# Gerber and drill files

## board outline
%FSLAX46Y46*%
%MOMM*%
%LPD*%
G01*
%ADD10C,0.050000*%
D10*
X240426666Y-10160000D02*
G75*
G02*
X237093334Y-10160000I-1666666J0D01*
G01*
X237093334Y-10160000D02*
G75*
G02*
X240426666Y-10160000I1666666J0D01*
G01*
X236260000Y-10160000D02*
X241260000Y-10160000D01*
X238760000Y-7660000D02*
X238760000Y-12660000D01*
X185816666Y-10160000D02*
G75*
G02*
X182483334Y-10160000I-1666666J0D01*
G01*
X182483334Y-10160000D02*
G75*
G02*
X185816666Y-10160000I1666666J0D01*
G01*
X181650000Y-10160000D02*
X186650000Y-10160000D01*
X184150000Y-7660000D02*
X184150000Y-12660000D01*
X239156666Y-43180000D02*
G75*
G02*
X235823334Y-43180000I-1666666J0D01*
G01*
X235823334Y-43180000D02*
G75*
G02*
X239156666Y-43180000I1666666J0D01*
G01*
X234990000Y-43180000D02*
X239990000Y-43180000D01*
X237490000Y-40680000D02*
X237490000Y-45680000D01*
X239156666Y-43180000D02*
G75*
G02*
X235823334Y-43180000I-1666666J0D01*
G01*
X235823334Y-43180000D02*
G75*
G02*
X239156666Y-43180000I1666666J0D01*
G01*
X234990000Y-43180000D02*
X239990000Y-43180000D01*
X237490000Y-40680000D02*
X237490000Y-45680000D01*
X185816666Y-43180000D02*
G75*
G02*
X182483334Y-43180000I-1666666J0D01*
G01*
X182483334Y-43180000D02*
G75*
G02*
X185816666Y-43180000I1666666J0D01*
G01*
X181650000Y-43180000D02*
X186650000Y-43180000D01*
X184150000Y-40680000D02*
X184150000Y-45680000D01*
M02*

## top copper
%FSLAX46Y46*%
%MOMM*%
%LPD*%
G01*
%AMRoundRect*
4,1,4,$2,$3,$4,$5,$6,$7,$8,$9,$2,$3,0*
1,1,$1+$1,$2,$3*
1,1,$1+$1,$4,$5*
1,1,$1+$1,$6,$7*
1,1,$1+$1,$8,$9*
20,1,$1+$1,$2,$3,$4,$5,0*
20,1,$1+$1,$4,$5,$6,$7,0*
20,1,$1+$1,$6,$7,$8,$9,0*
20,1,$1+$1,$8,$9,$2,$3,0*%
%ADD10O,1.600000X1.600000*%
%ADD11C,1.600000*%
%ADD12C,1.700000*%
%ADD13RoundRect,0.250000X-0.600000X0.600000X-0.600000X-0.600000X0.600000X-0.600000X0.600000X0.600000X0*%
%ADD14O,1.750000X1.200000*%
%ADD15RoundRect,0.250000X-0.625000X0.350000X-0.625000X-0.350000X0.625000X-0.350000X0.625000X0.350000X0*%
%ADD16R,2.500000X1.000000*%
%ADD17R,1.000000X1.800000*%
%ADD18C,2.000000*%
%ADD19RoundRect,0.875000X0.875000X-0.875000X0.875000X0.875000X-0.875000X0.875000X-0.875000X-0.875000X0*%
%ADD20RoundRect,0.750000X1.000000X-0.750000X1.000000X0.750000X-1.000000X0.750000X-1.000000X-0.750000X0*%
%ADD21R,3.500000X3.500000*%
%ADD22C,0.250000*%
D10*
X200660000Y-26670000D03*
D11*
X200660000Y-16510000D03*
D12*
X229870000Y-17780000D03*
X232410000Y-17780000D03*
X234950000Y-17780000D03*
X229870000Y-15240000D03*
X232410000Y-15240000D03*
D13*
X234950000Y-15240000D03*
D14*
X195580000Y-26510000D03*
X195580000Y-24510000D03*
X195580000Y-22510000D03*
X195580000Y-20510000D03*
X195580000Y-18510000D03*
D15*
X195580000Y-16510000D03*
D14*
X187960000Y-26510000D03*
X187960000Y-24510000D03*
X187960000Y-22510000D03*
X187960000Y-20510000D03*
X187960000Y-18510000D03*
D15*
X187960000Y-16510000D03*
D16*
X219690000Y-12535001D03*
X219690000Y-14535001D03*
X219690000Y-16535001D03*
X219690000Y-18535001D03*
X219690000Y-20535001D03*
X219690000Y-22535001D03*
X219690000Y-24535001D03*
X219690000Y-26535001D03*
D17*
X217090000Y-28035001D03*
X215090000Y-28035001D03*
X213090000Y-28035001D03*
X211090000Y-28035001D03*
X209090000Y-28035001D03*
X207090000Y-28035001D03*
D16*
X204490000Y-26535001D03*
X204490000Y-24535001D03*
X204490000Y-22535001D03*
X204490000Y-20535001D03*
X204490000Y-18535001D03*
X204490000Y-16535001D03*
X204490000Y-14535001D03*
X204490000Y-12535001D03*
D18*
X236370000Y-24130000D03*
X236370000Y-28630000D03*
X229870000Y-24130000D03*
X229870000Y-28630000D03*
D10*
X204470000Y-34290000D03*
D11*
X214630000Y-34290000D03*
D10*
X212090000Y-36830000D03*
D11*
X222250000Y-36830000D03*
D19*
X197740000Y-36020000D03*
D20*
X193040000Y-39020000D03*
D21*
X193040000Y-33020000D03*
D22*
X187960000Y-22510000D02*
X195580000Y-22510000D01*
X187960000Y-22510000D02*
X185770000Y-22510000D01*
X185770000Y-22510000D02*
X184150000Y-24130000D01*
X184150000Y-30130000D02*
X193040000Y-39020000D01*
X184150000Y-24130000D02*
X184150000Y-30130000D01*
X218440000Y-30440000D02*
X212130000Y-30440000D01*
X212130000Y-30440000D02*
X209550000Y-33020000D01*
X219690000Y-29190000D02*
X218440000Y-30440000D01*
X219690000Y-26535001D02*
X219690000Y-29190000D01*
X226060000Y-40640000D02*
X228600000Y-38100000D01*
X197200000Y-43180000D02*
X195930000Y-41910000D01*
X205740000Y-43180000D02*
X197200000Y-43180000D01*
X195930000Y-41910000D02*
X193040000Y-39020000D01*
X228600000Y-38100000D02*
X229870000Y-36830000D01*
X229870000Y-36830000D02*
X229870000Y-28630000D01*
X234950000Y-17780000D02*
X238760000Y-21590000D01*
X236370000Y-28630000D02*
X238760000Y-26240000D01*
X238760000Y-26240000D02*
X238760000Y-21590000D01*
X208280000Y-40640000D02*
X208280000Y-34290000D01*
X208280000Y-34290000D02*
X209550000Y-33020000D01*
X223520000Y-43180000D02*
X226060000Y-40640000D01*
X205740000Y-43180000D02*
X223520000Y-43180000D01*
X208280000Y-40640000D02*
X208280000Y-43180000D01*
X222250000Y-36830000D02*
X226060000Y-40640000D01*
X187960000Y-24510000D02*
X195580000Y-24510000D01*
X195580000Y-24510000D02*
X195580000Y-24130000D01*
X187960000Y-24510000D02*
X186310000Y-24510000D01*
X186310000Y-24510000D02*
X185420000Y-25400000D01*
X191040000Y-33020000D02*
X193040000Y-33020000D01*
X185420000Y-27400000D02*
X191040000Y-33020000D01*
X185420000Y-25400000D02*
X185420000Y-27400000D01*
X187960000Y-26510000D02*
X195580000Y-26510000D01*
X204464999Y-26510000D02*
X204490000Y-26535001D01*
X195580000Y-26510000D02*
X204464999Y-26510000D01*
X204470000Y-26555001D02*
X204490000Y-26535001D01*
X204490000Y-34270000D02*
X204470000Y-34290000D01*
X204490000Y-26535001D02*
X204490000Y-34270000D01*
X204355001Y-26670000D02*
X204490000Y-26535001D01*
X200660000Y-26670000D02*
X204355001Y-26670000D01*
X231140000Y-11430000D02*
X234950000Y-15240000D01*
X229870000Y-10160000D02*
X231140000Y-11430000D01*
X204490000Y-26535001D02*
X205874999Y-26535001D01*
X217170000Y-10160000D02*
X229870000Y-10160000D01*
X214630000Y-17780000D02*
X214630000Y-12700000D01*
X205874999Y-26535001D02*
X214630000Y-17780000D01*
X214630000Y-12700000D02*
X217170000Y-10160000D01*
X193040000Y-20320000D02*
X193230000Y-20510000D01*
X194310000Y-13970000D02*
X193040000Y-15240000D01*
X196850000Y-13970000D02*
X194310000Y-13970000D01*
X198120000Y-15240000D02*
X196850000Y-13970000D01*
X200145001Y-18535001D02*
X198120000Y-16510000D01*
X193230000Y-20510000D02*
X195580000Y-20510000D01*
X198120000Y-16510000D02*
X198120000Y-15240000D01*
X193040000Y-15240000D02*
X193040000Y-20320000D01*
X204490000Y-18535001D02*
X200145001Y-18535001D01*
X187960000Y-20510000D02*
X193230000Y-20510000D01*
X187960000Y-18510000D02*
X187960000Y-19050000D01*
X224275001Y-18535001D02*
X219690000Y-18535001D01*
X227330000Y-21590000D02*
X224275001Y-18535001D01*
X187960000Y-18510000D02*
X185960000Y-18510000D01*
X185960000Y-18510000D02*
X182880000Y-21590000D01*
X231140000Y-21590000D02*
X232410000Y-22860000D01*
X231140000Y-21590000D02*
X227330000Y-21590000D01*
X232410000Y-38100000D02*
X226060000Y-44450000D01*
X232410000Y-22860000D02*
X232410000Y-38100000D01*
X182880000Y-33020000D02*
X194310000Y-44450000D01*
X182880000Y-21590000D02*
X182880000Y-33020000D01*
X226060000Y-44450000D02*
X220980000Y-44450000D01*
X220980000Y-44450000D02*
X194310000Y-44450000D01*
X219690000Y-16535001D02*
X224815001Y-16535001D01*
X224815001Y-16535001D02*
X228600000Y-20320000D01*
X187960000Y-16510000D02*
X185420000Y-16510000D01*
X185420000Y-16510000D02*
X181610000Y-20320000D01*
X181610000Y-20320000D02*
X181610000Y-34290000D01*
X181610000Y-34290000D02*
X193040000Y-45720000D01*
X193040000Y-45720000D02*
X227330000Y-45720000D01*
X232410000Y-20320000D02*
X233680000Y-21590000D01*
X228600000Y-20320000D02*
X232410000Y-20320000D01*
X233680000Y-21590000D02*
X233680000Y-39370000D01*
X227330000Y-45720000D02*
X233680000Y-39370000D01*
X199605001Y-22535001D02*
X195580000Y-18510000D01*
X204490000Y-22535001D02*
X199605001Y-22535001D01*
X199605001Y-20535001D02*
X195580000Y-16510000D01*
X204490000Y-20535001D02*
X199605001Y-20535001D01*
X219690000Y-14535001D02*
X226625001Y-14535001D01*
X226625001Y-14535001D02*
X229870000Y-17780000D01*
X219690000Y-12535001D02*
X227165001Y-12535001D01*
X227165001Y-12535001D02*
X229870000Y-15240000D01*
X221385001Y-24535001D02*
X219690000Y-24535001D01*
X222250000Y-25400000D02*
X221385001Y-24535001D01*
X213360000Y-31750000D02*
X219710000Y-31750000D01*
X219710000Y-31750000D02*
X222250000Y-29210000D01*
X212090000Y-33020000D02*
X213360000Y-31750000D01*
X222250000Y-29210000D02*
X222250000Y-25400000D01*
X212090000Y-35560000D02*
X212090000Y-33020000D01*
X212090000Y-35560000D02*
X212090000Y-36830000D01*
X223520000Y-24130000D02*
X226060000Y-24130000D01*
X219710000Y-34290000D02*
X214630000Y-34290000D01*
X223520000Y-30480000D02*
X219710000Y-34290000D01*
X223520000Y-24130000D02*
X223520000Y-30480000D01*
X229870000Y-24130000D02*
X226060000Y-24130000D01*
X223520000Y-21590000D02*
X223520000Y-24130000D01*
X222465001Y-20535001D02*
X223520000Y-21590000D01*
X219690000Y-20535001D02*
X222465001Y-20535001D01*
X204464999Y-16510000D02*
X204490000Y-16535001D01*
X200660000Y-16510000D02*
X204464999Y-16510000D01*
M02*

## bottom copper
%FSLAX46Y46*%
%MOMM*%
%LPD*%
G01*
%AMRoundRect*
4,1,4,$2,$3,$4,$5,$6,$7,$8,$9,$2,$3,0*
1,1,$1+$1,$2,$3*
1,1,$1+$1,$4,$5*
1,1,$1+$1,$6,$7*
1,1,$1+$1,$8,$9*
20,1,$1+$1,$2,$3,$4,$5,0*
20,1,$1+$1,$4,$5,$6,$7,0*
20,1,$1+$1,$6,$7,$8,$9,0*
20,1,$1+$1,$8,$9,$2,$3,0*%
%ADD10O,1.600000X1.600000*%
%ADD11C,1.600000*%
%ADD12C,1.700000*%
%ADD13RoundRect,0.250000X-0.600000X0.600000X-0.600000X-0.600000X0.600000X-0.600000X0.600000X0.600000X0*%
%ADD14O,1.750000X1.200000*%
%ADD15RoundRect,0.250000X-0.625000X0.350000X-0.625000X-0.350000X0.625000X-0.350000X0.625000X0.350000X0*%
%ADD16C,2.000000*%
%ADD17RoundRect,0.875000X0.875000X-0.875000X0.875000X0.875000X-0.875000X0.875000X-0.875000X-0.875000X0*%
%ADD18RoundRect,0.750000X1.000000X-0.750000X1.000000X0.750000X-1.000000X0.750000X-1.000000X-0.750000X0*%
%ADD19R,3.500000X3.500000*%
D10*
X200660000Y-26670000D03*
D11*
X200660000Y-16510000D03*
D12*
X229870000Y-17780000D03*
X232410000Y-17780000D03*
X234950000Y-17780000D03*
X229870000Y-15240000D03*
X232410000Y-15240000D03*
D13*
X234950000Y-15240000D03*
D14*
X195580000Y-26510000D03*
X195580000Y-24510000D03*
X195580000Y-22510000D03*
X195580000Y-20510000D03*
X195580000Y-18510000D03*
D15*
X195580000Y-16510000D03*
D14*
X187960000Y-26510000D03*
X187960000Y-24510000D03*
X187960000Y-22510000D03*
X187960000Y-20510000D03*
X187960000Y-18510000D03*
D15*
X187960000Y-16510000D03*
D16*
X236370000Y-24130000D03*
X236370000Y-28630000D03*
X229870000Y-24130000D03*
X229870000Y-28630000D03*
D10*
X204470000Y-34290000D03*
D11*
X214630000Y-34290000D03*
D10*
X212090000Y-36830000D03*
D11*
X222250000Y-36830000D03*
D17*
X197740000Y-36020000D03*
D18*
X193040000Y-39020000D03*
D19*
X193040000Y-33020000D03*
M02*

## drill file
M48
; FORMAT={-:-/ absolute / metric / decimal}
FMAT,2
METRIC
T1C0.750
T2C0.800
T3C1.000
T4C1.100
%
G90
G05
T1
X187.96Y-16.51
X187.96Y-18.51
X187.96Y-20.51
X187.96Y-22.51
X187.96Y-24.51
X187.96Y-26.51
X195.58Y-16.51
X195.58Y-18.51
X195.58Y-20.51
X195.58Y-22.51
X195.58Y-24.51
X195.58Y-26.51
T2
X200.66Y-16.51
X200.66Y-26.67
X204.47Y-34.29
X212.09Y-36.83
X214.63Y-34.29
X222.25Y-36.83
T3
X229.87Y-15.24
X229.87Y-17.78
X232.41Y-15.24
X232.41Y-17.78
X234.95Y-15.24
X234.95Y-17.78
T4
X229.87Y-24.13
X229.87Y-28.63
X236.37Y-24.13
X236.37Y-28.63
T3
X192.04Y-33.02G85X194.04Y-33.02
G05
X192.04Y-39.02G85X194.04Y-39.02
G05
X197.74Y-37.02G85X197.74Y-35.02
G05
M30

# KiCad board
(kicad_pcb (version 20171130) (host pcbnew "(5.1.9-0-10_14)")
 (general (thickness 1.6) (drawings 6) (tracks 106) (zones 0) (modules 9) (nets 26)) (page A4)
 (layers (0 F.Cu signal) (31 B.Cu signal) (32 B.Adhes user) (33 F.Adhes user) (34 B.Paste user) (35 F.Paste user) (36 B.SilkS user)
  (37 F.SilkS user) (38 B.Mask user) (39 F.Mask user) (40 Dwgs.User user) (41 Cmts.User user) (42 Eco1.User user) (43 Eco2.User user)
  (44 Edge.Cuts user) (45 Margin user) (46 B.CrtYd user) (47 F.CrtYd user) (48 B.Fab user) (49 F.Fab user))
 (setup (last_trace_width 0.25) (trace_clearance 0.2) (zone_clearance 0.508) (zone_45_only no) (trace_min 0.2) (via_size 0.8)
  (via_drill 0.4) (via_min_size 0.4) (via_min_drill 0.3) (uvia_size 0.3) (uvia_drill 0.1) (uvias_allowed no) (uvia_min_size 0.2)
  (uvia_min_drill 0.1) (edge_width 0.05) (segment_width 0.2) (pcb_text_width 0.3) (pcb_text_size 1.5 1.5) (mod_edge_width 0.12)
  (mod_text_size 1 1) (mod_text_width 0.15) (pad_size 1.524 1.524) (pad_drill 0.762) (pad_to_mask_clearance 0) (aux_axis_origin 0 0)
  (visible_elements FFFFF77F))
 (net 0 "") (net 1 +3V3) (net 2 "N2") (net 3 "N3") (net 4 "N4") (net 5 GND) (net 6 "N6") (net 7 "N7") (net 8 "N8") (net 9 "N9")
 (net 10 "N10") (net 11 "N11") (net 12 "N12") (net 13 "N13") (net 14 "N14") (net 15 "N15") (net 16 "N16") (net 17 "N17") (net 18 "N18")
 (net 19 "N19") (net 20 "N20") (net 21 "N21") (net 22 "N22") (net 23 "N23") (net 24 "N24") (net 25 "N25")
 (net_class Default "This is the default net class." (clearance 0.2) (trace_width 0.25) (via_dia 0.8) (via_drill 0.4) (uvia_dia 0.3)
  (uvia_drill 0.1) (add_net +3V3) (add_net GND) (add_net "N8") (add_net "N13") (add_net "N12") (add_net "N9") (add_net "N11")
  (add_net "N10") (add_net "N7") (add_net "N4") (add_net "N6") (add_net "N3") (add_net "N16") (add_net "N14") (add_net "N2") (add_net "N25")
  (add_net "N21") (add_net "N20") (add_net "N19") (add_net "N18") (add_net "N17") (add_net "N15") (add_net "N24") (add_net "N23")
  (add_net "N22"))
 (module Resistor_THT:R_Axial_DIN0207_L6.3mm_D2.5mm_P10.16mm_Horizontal (layer F.Cu) (at 200.66 16.51 270)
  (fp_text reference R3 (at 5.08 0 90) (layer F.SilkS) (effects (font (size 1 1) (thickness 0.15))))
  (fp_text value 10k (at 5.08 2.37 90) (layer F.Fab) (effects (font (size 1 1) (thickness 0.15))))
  (pad 2 thru_hole oval (at 10.16 0 270) (size 1.6 1.6) (drill 0.8) (layers *.Cu *.Mask) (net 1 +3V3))
  (pad 1 thru_hole circle (at 0 0 270) (size 1.6 1.6) (drill 0.8) (layers *.Cu *.Mask) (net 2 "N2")))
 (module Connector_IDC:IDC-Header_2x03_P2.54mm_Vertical (layer F.Cu) (at 234.95 15.24 270)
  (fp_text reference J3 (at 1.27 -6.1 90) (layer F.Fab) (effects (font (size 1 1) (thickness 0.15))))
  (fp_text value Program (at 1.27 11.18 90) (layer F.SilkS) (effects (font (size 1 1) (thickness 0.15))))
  (pad 6 thru_hole circle (at 2.54 5.08 270) (size 1.7 1.7) (drill 1) (layers *.Cu *.Mask) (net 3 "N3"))
  (pad 4 thru_hole circle (at 2.54 2.54 270) (size 1.7 1.7) (drill 1) (layers *.Cu *.Mask) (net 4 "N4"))
  (pad 2 thru_hole circle (at 2.54 0 270) (size 1.7 1.7) (drill 1) (layers *.Cu *.Mask) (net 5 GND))
  (pad 5 thru_hole circle (at 0 5.08 270) (size 1.7 1.7) (drill 1) (layers *.Cu *.Mask) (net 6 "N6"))
  (pad 3 thru_hole circle (at 0 2.54 270) (size 1.7 1.7) (drill 1) (layers *.Cu *.Mask) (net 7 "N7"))
  (pad 1 thru_hole roundrect (at 0 0 270) (size 1.7 1.7) (drill 1) (layers *.Cu *.Mask) (roundrect_rratio 0.147059) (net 1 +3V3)))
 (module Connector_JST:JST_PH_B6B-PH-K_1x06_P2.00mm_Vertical (layer F.Cu) (at 195.58 16.51 270)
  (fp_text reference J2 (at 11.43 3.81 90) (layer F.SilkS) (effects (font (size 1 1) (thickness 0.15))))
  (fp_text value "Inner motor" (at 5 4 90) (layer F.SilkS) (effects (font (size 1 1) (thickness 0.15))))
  (pad 6 thru_hole oval (at 10 0 270) (size 1.2 1.75) (drill 0.75) (layers *.Cu *.Mask) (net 1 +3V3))
  (pad 5 thru_hole oval (at 8 0 270) (size 1.2 1.75) (drill 0.75) (layers *.Cu *.Mask) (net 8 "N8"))
  (pad 4 thru_hole oval (at 6 0 270) (size 1.2 1.75) (drill 0.75) (layers *.Cu *.Mask) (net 5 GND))
  (pad 3 thru_hole oval (at 4 0 270) (size 1.2 1.75) (drill 0.75) (layers *.Cu *.Mask) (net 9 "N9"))
  (pad 2 thru_hole oval (at 2 0 270) (size 1.2 1.75) (drill 0.75) (layers *.Cu *.Mask) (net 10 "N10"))
  (pad 1 thru_hole roundrect (at 0 0 270) (size 1.2 1.75) (drill 0.75) (layers *.Cu *.Mask) (roundrect_rratio 0.208333) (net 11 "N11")))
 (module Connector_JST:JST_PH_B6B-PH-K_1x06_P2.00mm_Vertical (layer F.Cu) (at 187.96 16.51 270)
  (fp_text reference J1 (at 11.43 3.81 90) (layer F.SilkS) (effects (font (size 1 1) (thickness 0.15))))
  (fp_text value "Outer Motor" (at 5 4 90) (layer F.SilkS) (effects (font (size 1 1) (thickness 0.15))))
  (pad 6 thru_hole oval (at 10 0 270) (size 1.2 1.75) (drill 0.75) (layers *.Cu *.Mask) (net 1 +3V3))
  (pad 5 thru_hole oval (at 8 0 270) (size 1.2 1.75) (drill 0.75) (layers *.Cu *.Mask) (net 8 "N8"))
  (pad 4 thru_hole oval (at 6 0 270) (size 1.2 1.75) (drill 0.75) (layers *.Cu *.Mask) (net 5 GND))
  (pad 3 thru_hole oval (at 4 0 270) (size 1.2 1.75) (drill 0.75) (layers *.Cu *.Mask) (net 9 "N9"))
  (pad 2 thru_hole oval (at 2 0 270) (size 1.2 1.75) (drill 0.75) (layers *.Cu *.Mask) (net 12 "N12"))
  (pad 1 thru_hole roundrect (at 0 0 270) (size 1.2 1.75) (drill 0.75) (layers *.Cu *.Mask) (roundrect_rratio 0.208333) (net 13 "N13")))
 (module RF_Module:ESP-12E (layer F.Cu) (at 212.09 16.035001)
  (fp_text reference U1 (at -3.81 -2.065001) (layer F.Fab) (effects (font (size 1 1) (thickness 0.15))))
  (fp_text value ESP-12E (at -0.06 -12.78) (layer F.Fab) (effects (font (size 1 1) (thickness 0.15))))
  (pad 22 smd rect (at 7.6 -3.5) (size 2.5 1) (layers F.Cu F.Paste F.Mask) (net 6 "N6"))
  (pad 21 smd rect (at 7.6 -1.5) (size 2.5 1) (layers F.Cu F.Paste F.Mask) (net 3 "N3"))
  (pad 20 smd rect (at 7.6 0.5) (size 2.5 1) (layers F.Cu F.Paste F.Mask) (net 13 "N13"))
  (pad 19 smd rect (at 7.6 2.5) (size 2.5 1) (layers F.Cu F.Paste F.Mask) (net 12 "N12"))
  (pad 18 smd rect (at 7.6 4.5) (size 2.5 1) (layers F.Cu F.Paste F.Mask) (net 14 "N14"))
  (pad 17 smd rect (at 7.6 6.5) (size 2.5 1) (layers F.Cu F.Paste F.Mask) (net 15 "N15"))
  (pad 16 smd rect (at 7.6 8.5) (size 2.5 1) (layers F.Cu F.Paste F.Mask) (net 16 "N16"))
  (pad 15 smd rect (at 7.6 10.5) (size 2.5 1) (layers F.Cu F.Paste F.Mask) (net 5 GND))
  (pad 14 smd rect (at 5 12) (size 1 1.8) (layers F.Cu F.Paste F.Mask) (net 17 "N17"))
  (pad 13 smd rect (at 3 12) (size 1 1.8) (layers F.Cu F.Paste F.Mask) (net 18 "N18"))
  (pad 12 smd rect (at 1 12) (size 1 1.8) (layers F.Cu F.Paste F.Mask) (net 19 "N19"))
  (pad 11 smd rect (at -1 12) (size 1 1.8) (layers F.Cu F.Paste F.Mask) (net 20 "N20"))
  (pad 10 smd rect (at -3 12) (size 1 1.8) (layers F.Cu F.Paste F.Mask) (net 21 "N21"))
  (pad 9 smd rect (at -5 12) (size 1 1.8) (layers F.Cu F.Paste F.Mask) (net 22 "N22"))
  (pad 8 smd rect (at -7.6 10.5) (size 2.5 1) (layers F.Cu F.Paste F.Mask) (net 1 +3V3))
  (pad 7 smd rect (at -7.6 8.5) (size 2.5 1) (layers F.Cu F.Paste F.Mask) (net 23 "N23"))
  (pad 6 smd rect (at -7.6 6.5) (size 2.5 1) (layers F.Cu F.Paste F.Mask) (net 10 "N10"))
  (pad 5 smd rect (at -7.6 4.5) (size 2.5 1) (layers F.Cu F.Paste F.Mask) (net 11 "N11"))
  (pad 4 smd rect (at -7.6 2.5) (size 2.5 1) (layers F.Cu F.Paste F.Mask) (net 9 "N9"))
  (pad 3 smd rect (at -7.6 0.5) (size 2.5 1) (layers F.Cu F.Paste F.Mask) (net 2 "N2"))
  (pad 2 smd rect (at -7.6 -1.5) (size 2.5 1) (layers F.Cu F.Paste F.Mask) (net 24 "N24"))
  (pad 1 smd rect (at -7.6 -3.5) (size 2.5 1) (layers F.Cu F.Paste F.Mask) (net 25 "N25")))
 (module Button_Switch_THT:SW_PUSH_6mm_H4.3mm (layer F.Cu) (at 229.87 24.13)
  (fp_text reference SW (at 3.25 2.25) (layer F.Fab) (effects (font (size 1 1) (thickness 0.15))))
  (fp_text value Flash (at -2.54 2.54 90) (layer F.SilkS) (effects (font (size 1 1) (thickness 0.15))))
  (pad 1 thru_hole circle (at 6.5 0 90) (size 2 2) (drill 1.1) (layers *.Cu *.Mask) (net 14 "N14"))
  (pad 2 thru_hole circle (at 6.5 4.5 90) (size 2 2) (drill 1.1) (layers *.Cu *.Mask) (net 5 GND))
  (pad 1 thru_hole circle (at 0 0 90) (size 2 2) (drill 1.1) (layers *.Cu *.Mask) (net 14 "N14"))
  (pad 2 thru_hole circle (at 0 4.5 90) (size 2 2) (drill 1.1) (layers *.Cu *.Mask) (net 5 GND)))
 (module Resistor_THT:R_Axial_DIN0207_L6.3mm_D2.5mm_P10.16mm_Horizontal (layer F.Cu) (at 214.63 34.29 180)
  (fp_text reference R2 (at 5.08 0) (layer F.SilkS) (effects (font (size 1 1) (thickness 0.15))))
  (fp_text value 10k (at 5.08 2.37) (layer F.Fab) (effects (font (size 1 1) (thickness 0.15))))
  (pad 2 thru_hole oval (at 10.16 0 180) (size 1.6 1.6) (drill 0.8) (layers *.Cu *.Mask) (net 1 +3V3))
  (pad 1 thru_hole circle (at 0 0 180) (size 1.6 1.6) (drill 0.8) (layers *.Cu *.Mask) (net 14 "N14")))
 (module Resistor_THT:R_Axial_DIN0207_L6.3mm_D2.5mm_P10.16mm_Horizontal (layer F.Cu) (at 222.25 36.83 180)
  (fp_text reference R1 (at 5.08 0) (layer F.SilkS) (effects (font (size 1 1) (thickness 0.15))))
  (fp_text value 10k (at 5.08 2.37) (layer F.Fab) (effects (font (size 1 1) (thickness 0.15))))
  (pad 2 thru_hole oval (at 10.16 0 180) (size 1.6 1.6) (drill 0.8) (layers *.Cu *.Mask) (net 16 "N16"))
  (pad 1 thru_hole circle (at 0 0 180) (size 1.6 1.6) (drill 0.8) (layers *.Cu *.Mask) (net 5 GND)))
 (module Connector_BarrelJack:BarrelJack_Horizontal (layer F.Cu) (at 193.04 33.02 90)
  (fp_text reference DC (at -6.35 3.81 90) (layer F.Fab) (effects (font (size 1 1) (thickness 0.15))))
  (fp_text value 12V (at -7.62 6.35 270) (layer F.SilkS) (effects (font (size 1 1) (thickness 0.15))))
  (pad 3 thru_hole roundrect (at -3 4.7 90) (size 3.5 3.5) (drill oval 3 1) (layers *.Cu *.Mask) (roundrect_rratio 0.25))
  (pad 2 thru_hole roundrect (at -6 0 90) (size 3 3.5) (drill oval 1 3) (layers *.Cu *.Mask) (roundrect_rratio 0.25) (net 5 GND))
  (pad 1 thru_hole rect (at 0 0 90) (size 3.5 3.5) (drill oval 1 3) (layers *.Cu *.Mask) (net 8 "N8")))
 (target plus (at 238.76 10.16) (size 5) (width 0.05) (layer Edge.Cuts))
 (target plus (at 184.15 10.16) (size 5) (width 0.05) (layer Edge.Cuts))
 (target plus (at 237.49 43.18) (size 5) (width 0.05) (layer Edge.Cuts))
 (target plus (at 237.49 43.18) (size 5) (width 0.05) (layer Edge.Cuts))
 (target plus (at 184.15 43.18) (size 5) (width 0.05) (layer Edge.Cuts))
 (segment (start 187.96 22.51) (end 195.58 22.51) (width 0.25) (layer F.Cu) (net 5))
 (segment (start 187.96 22.51) (end 185.77 22.51) (width 0.25) (layer F.Cu) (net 5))
 (segment (start 185.77 22.51) (end 184.15 24.13) (width 0.25) (layer F.Cu) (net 5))
 (segment (start 184.15 30.13) (end 193.04 39.02) (width 0.25) (layer F.Cu) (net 5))
 (segment (start 184.15 24.13) (end 184.15 30.13) (width 0.25) (layer F.Cu) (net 5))
 (segment (start 218.44 30.44) (end 212.13 30.44) (width 0.25) (layer F.Cu) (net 5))
 (segment (start 212.13 30.44) (end 209.55 33.02) (width 0.25) (layer F.Cu) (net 5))
 (segment (start 219.69 29.19) (end 218.44 30.44) (width 0.25) (layer F.Cu) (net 5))
 (segment (start 219.69 26.535001) (end 219.69 29.19) (width 0.25) (layer F.Cu) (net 5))
 (segment (start 226.06 40.64) (end 228.6 38.1) (width 0.25) (layer F.Cu) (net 5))
 (segment (start 197.2 43.18) (end 195.93 41.91) (width 0.25) (layer F.Cu) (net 5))
 (segment (start 205.74 43.18) (end 197.2 43.18) (width 0.25) (layer F.Cu) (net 5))
 (segment (start 195.93 41.91) (end 193.04 39.02) (width 0.25) (layer F.Cu) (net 5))
 (segment (start 228.6 38.1) (end 229.87 36.83) (width 0.25) (layer F.Cu) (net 5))
 (segment (start 229.87 36.83) (end 229.87 28.63) (width 0.25) (layer F.Cu) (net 5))
 (segment (start 234.95 17.78) (end 238.76 21.59) (width 0.25) (layer F.Cu) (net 5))
 (segment (start 236.37 28.63) (end 238.76 26.24) (width 0.25) (layer F.Cu) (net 5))
 (segment (start 238.76 26.24) (end 238.76 21.59) (width 0.25) (layer F.Cu) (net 5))
 (segment (start 208.28 40.64) (end 208.28 34.29) (width 0.25) (layer F.Cu) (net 5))
 (segment (start 208.28 34.29) (end 209.55 33.02) (width 0.25) (layer F.Cu) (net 5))
 (segment (start 223.52 43.18) (end 226.06 40.64) (width 0.25) (layer F.Cu) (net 5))
 (segment (start 205.74 43.18) (end 223.52 43.18) (width 0.25) (layer F.Cu) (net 5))
 (segment (start 208.28 40.64) (end 208.28 43.18) (width 0.25) (layer F.Cu) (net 5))
 (segment (start 222.25 36.83) (end 226.06 40.64) (width 0.25) (layer F.Cu) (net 5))
 (segment (start 187.96 24.51) (end 195.58 24.51) (width 0.25) (layer F.Cu) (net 8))
 (segment (start 195.58 24.51) (end 195.58 24.13) (width 0.25) (layer F.Cu) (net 8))
 (segment (start 187.96 24.51) (end 186.31 24.51) (width 0.25) (layer F.Cu) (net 8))
 (segment (start 186.31 24.51) (end 185.42 25.4) (width 0.25) (layer F.Cu) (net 8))
 (segment (start 191.04 33.02) (end 193.04 33.02) (width 0.25) (layer F.Cu) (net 8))
 (segment (start 185.42 27.4) (end 191.04 33.02) (width 0.25) (layer F.Cu) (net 8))
 (segment (start 185.42 25.4) (end 185.42 27.4) (width 0.25) (layer F.Cu) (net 8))
 (segment (start 187.96 26.51) (end 195.58 26.51) (width 0.25) (layer F.Cu) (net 1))
 (segment (start 204.464999 26.51) (end 204.49 26.535001) (width 0.25) (layer F.Cu) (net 1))
 (segment (start 195.58 26.51) (end 204.464999 26.51) (width 0.25) (layer F.Cu) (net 1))
 (segment (start 204.47 26.555001) (end 204.49 26.535001) (width 0.25) (layer F.Cu) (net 1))
 (segment (start 204.49 34.27) (end 204.47 34.29) (width 0.25) (layer F.Cu) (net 1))
 (segment (start 204.49 26.535001) (end 204.49 34.27) (width 0.25) (layer F.Cu) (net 1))
 (segment (start 204.355001 26.67) (end 204.49 26.535001) (width 0.25) (layer F.Cu) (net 1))
 (segment (start 200.66 26.67) (end 204.355001 26.67) (width 0.25) (layer F.Cu) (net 1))
 (segment (start 231.14 11.43) (end 234.95 15.24) (width 0.25) (layer F.Cu) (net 1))
 (segment (start 229.87 10.16) (end 231.14 11.43) (width 0.25) (layer F.Cu) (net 1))
 (segment (start 204.49 26.535001) (end 205.874999 26.535001) (width 0.25) (layer F.Cu) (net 1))
 (segment (start 217.17 10.16) (end 229.87 10.16) (width 0.25) (layer F.Cu) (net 1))
 (segment (start 214.63 17.78) (end 214.63 12.7) (width 0.25) (layer F.Cu) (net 1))
 (segment (start 205.874999 26.535001) (end 214.63 17.78) (width 0.25) (layer F.Cu) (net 1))
 (segment (start 214.63 12.7) (end 217.17 10.16) (width 0.25) (layer F.Cu) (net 1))
 (segment (start 193.04 20.32) (end 193.23 20.51) (width 0.25) (layer F.Cu) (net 9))
 (segment (start 194.31 13.97) (end 193.04 15.24) (width 0.25) (layer F.Cu) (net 9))
 (segment (start 196.85 13.97) (end 194.31 13.97) (width 0.25) (layer F.Cu) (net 9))
 (segment (start 198.12 15.24) (end 196.85 13.97) (width 0.25) (layer F.Cu) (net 9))
 (segment (start 200.145001 18.535001) (end 198.12 16.51) (width 0.25) (layer F.Cu) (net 9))
 (segment (start 193.23 20.51) (end 195.58 20.51) (width 0.25) (layer F.Cu) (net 9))
 (segment (start 198.12 16.51) (end 198.12 15.24) (width 0.25) (layer F.Cu) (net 9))
 (segment (start 193.04 15.24) (end 193.04 20.32) (width 0.25) (layer F.Cu) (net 9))
 (segment (start 204.49 18.535001) (end 200.145001 18.535001) (width 0.25) (layer F.Cu) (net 9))
 (segment (start 187.96 20.51) (end 193.23 20.51) (width 0.25) (layer F.Cu) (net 9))
 (segment (start 187.96 18.51) (end 187.96 19.05) (width 0.25) (layer F.Cu) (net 12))
 (segment (start 224.275001 18.535001) (end 219.69 18.535001) (width 0.25) (layer F.Cu) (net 12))
 (segment (start 227.33 21.59) (end 224.275001 18.535001) (width 0.25) (layer F.Cu) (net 12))
 (segment (start 187.96 18.51) (end 185.96 18.51) (width 0.25) (layer F.Cu) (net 12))
 (segment (start 185.96 18.51) (end 182.88 21.59) (width 0.25) (layer F.Cu) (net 12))
 (segment (start 231.14 21.59) (end 232.41 22.86) (width 0.25) (layer F.Cu) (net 12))
 (segment (start 231.14 21.59) (end 227.33 21.59) (width 0.25) (layer F.Cu) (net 12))
 (segment (start 232.41 38.1) (end 226.06 44.45) (width 0.25) (layer F.Cu) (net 12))
 (segment (start 232.41 22.86) (end 232.41 38.1) (width 0.25) (layer F.Cu) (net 12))
 (segment (start 182.88 33.02) (end 194.31 44.45) (width 0.25) (layer F.Cu) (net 12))
 (segment (start 182.88 21.59) (end 182.88 33.02) (width 0.25) (layer F.Cu) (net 12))
 (segment (start 226.06 44.45) (end 220.98 44.45) (width 0.25) (layer F.Cu) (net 12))
 (segment (start 220.98 44.45) (end 194.31 44.45) (width 0.25) (layer F.Cu) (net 12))
 (segment (start 219.69 16.535001) (end 224.815001 16.535001) (width 0.25) (layer F.Cu) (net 13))
 (segment (start 224.815001 16.535001) (end 228.6 20.32) (width 0.25) (layer F.Cu) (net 13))
 (segment (start 187.96 16.51) (end 185.42 16.51) (width 0.25) (layer F.Cu) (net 13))
 (segment (start 185.42 16.51) (end 181.61 20.32) (width 0.25) (layer F.Cu) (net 13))
 (segment (start 181.61 20.32) (end 181.61 34.29) (width 0.25) (layer F.Cu) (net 13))
 (segment (start 181.61 34.29) (end 193.04 45.72) (width 0.25) (layer F.Cu) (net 13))
 (segment (start 193.04 45.72) (end 227.33 45.72) (width 0.25) (layer F.Cu) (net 13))
 (segment (start 232.41 20.32) (end 233.68 21.59) (width 0.25) (layer F.Cu) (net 13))
 (segment (start 228.6 20.32) (end 232.41 20.32) (width 0.25) (layer F.Cu) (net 13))
 (segment (start 233.68 21.59) (end 233.68 39.37) (width 0.25) (layer F.Cu) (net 13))
 (segment (start 227.33 45.72) (end 233.68 39.37) (width 0.25) (layer F.Cu) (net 13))
 (segment (start 199.605001 22.535001) (end 195.58 18.51) (width 0.25) (layer F.Cu) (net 10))
 (segment (start 204.49 22.535001) (end 199.605001 22.535001) (width 0.25) (layer F.Cu) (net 10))
 (segment (start 199.605001 20.535001) (end 195.58 16.51) (width 0.25) (layer F.Cu) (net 11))
 (segment (start 204.49 20.535001) (end 199.605001 20.535001) (width 0.25) (layer F.Cu) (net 11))
 (segment (start 219.69 14.535001) (end 226.625001 14.535001) (width 0.25) (layer F.Cu) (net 3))
 (segment (start 226.625001 14.535001) (end 229.87 17.78) (width 0.25) (layer F.Cu) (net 3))
 (segment (start 219.69 12.535001) (end 227.165001 12.535001) (width 0.25) (layer F.Cu) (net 6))
 (segment (start 227.165001 12.535001) (end 229.87 15.24) (width 0.25) (layer F.Cu) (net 6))
 (segment (start 221.385001 24.535001) (end 219.69 24.535001) (width 0.25) (layer F.Cu) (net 16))
 (segment (start 222.25 25.4) (end 221.385001 24.535001) (width 0.25) (layer F.Cu) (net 16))
 (segment (start 213.36 31.75) (end 219.71 31.75) (width 0.25) (layer F.Cu) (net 16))
 (segment (start 219.71 31.75) (end 222.25 29.21) (width 0.25) (layer F.Cu) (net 16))
 (segment (start 212.09 33.02) (end 213.36 31.75) (width 0.25) (layer F.Cu) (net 16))
 (segment (start 222.25 29.21) (end 222.25 25.4) (width 0.25) (layer F.Cu) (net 16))
 (segment (start 212.09 35.56) (end 212.09 33.02) (width 0.25) (layer F.Cu) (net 16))
 (segment (start 212.09 35.56) (end 212.09 36.83) (width 0.25) (layer F.Cu) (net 16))
 (segment (start 223.52 24.13) (end 226.06 24.13) (width 0.25) (layer F.Cu) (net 14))
 (segment (start 219.71 34.29) (end 214.63 34.29) (width 0.25) (layer F.Cu) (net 14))
 (segment (start 223.52 30.48) (end 219.71 34.29) (width 0.25) (layer F.Cu) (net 14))
 (segment (start 223.52 24.13) (end 223.52 30.48) (width 0.25) (layer F.Cu) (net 14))
 (segment (start 229.87 24.13) (end 226.06 24.13) (width 0.25) (layer F.Cu) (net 14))
 (segment (start 223.52 21.59) (end 223.52 24.13) (width 0.25) (layer F.Cu) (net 14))
 (segment (start 222.465001 20.535001) (end 223.52 21.59) (width 0.25) (layer F.Cu) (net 14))
 (segment (start 219.69 20.535001) (end 222.465001 20.535001) (width 0.25) (layer F.Cu) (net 14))
 (segment (start 204.464999 16.51) (end 204.49 16.535001) (width 0.25) (layer F.Cu) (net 2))
 (segment (start 200.66 16.51) (end 204.464999 16.51) (width 0.25) (layer F.Cu) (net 2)))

